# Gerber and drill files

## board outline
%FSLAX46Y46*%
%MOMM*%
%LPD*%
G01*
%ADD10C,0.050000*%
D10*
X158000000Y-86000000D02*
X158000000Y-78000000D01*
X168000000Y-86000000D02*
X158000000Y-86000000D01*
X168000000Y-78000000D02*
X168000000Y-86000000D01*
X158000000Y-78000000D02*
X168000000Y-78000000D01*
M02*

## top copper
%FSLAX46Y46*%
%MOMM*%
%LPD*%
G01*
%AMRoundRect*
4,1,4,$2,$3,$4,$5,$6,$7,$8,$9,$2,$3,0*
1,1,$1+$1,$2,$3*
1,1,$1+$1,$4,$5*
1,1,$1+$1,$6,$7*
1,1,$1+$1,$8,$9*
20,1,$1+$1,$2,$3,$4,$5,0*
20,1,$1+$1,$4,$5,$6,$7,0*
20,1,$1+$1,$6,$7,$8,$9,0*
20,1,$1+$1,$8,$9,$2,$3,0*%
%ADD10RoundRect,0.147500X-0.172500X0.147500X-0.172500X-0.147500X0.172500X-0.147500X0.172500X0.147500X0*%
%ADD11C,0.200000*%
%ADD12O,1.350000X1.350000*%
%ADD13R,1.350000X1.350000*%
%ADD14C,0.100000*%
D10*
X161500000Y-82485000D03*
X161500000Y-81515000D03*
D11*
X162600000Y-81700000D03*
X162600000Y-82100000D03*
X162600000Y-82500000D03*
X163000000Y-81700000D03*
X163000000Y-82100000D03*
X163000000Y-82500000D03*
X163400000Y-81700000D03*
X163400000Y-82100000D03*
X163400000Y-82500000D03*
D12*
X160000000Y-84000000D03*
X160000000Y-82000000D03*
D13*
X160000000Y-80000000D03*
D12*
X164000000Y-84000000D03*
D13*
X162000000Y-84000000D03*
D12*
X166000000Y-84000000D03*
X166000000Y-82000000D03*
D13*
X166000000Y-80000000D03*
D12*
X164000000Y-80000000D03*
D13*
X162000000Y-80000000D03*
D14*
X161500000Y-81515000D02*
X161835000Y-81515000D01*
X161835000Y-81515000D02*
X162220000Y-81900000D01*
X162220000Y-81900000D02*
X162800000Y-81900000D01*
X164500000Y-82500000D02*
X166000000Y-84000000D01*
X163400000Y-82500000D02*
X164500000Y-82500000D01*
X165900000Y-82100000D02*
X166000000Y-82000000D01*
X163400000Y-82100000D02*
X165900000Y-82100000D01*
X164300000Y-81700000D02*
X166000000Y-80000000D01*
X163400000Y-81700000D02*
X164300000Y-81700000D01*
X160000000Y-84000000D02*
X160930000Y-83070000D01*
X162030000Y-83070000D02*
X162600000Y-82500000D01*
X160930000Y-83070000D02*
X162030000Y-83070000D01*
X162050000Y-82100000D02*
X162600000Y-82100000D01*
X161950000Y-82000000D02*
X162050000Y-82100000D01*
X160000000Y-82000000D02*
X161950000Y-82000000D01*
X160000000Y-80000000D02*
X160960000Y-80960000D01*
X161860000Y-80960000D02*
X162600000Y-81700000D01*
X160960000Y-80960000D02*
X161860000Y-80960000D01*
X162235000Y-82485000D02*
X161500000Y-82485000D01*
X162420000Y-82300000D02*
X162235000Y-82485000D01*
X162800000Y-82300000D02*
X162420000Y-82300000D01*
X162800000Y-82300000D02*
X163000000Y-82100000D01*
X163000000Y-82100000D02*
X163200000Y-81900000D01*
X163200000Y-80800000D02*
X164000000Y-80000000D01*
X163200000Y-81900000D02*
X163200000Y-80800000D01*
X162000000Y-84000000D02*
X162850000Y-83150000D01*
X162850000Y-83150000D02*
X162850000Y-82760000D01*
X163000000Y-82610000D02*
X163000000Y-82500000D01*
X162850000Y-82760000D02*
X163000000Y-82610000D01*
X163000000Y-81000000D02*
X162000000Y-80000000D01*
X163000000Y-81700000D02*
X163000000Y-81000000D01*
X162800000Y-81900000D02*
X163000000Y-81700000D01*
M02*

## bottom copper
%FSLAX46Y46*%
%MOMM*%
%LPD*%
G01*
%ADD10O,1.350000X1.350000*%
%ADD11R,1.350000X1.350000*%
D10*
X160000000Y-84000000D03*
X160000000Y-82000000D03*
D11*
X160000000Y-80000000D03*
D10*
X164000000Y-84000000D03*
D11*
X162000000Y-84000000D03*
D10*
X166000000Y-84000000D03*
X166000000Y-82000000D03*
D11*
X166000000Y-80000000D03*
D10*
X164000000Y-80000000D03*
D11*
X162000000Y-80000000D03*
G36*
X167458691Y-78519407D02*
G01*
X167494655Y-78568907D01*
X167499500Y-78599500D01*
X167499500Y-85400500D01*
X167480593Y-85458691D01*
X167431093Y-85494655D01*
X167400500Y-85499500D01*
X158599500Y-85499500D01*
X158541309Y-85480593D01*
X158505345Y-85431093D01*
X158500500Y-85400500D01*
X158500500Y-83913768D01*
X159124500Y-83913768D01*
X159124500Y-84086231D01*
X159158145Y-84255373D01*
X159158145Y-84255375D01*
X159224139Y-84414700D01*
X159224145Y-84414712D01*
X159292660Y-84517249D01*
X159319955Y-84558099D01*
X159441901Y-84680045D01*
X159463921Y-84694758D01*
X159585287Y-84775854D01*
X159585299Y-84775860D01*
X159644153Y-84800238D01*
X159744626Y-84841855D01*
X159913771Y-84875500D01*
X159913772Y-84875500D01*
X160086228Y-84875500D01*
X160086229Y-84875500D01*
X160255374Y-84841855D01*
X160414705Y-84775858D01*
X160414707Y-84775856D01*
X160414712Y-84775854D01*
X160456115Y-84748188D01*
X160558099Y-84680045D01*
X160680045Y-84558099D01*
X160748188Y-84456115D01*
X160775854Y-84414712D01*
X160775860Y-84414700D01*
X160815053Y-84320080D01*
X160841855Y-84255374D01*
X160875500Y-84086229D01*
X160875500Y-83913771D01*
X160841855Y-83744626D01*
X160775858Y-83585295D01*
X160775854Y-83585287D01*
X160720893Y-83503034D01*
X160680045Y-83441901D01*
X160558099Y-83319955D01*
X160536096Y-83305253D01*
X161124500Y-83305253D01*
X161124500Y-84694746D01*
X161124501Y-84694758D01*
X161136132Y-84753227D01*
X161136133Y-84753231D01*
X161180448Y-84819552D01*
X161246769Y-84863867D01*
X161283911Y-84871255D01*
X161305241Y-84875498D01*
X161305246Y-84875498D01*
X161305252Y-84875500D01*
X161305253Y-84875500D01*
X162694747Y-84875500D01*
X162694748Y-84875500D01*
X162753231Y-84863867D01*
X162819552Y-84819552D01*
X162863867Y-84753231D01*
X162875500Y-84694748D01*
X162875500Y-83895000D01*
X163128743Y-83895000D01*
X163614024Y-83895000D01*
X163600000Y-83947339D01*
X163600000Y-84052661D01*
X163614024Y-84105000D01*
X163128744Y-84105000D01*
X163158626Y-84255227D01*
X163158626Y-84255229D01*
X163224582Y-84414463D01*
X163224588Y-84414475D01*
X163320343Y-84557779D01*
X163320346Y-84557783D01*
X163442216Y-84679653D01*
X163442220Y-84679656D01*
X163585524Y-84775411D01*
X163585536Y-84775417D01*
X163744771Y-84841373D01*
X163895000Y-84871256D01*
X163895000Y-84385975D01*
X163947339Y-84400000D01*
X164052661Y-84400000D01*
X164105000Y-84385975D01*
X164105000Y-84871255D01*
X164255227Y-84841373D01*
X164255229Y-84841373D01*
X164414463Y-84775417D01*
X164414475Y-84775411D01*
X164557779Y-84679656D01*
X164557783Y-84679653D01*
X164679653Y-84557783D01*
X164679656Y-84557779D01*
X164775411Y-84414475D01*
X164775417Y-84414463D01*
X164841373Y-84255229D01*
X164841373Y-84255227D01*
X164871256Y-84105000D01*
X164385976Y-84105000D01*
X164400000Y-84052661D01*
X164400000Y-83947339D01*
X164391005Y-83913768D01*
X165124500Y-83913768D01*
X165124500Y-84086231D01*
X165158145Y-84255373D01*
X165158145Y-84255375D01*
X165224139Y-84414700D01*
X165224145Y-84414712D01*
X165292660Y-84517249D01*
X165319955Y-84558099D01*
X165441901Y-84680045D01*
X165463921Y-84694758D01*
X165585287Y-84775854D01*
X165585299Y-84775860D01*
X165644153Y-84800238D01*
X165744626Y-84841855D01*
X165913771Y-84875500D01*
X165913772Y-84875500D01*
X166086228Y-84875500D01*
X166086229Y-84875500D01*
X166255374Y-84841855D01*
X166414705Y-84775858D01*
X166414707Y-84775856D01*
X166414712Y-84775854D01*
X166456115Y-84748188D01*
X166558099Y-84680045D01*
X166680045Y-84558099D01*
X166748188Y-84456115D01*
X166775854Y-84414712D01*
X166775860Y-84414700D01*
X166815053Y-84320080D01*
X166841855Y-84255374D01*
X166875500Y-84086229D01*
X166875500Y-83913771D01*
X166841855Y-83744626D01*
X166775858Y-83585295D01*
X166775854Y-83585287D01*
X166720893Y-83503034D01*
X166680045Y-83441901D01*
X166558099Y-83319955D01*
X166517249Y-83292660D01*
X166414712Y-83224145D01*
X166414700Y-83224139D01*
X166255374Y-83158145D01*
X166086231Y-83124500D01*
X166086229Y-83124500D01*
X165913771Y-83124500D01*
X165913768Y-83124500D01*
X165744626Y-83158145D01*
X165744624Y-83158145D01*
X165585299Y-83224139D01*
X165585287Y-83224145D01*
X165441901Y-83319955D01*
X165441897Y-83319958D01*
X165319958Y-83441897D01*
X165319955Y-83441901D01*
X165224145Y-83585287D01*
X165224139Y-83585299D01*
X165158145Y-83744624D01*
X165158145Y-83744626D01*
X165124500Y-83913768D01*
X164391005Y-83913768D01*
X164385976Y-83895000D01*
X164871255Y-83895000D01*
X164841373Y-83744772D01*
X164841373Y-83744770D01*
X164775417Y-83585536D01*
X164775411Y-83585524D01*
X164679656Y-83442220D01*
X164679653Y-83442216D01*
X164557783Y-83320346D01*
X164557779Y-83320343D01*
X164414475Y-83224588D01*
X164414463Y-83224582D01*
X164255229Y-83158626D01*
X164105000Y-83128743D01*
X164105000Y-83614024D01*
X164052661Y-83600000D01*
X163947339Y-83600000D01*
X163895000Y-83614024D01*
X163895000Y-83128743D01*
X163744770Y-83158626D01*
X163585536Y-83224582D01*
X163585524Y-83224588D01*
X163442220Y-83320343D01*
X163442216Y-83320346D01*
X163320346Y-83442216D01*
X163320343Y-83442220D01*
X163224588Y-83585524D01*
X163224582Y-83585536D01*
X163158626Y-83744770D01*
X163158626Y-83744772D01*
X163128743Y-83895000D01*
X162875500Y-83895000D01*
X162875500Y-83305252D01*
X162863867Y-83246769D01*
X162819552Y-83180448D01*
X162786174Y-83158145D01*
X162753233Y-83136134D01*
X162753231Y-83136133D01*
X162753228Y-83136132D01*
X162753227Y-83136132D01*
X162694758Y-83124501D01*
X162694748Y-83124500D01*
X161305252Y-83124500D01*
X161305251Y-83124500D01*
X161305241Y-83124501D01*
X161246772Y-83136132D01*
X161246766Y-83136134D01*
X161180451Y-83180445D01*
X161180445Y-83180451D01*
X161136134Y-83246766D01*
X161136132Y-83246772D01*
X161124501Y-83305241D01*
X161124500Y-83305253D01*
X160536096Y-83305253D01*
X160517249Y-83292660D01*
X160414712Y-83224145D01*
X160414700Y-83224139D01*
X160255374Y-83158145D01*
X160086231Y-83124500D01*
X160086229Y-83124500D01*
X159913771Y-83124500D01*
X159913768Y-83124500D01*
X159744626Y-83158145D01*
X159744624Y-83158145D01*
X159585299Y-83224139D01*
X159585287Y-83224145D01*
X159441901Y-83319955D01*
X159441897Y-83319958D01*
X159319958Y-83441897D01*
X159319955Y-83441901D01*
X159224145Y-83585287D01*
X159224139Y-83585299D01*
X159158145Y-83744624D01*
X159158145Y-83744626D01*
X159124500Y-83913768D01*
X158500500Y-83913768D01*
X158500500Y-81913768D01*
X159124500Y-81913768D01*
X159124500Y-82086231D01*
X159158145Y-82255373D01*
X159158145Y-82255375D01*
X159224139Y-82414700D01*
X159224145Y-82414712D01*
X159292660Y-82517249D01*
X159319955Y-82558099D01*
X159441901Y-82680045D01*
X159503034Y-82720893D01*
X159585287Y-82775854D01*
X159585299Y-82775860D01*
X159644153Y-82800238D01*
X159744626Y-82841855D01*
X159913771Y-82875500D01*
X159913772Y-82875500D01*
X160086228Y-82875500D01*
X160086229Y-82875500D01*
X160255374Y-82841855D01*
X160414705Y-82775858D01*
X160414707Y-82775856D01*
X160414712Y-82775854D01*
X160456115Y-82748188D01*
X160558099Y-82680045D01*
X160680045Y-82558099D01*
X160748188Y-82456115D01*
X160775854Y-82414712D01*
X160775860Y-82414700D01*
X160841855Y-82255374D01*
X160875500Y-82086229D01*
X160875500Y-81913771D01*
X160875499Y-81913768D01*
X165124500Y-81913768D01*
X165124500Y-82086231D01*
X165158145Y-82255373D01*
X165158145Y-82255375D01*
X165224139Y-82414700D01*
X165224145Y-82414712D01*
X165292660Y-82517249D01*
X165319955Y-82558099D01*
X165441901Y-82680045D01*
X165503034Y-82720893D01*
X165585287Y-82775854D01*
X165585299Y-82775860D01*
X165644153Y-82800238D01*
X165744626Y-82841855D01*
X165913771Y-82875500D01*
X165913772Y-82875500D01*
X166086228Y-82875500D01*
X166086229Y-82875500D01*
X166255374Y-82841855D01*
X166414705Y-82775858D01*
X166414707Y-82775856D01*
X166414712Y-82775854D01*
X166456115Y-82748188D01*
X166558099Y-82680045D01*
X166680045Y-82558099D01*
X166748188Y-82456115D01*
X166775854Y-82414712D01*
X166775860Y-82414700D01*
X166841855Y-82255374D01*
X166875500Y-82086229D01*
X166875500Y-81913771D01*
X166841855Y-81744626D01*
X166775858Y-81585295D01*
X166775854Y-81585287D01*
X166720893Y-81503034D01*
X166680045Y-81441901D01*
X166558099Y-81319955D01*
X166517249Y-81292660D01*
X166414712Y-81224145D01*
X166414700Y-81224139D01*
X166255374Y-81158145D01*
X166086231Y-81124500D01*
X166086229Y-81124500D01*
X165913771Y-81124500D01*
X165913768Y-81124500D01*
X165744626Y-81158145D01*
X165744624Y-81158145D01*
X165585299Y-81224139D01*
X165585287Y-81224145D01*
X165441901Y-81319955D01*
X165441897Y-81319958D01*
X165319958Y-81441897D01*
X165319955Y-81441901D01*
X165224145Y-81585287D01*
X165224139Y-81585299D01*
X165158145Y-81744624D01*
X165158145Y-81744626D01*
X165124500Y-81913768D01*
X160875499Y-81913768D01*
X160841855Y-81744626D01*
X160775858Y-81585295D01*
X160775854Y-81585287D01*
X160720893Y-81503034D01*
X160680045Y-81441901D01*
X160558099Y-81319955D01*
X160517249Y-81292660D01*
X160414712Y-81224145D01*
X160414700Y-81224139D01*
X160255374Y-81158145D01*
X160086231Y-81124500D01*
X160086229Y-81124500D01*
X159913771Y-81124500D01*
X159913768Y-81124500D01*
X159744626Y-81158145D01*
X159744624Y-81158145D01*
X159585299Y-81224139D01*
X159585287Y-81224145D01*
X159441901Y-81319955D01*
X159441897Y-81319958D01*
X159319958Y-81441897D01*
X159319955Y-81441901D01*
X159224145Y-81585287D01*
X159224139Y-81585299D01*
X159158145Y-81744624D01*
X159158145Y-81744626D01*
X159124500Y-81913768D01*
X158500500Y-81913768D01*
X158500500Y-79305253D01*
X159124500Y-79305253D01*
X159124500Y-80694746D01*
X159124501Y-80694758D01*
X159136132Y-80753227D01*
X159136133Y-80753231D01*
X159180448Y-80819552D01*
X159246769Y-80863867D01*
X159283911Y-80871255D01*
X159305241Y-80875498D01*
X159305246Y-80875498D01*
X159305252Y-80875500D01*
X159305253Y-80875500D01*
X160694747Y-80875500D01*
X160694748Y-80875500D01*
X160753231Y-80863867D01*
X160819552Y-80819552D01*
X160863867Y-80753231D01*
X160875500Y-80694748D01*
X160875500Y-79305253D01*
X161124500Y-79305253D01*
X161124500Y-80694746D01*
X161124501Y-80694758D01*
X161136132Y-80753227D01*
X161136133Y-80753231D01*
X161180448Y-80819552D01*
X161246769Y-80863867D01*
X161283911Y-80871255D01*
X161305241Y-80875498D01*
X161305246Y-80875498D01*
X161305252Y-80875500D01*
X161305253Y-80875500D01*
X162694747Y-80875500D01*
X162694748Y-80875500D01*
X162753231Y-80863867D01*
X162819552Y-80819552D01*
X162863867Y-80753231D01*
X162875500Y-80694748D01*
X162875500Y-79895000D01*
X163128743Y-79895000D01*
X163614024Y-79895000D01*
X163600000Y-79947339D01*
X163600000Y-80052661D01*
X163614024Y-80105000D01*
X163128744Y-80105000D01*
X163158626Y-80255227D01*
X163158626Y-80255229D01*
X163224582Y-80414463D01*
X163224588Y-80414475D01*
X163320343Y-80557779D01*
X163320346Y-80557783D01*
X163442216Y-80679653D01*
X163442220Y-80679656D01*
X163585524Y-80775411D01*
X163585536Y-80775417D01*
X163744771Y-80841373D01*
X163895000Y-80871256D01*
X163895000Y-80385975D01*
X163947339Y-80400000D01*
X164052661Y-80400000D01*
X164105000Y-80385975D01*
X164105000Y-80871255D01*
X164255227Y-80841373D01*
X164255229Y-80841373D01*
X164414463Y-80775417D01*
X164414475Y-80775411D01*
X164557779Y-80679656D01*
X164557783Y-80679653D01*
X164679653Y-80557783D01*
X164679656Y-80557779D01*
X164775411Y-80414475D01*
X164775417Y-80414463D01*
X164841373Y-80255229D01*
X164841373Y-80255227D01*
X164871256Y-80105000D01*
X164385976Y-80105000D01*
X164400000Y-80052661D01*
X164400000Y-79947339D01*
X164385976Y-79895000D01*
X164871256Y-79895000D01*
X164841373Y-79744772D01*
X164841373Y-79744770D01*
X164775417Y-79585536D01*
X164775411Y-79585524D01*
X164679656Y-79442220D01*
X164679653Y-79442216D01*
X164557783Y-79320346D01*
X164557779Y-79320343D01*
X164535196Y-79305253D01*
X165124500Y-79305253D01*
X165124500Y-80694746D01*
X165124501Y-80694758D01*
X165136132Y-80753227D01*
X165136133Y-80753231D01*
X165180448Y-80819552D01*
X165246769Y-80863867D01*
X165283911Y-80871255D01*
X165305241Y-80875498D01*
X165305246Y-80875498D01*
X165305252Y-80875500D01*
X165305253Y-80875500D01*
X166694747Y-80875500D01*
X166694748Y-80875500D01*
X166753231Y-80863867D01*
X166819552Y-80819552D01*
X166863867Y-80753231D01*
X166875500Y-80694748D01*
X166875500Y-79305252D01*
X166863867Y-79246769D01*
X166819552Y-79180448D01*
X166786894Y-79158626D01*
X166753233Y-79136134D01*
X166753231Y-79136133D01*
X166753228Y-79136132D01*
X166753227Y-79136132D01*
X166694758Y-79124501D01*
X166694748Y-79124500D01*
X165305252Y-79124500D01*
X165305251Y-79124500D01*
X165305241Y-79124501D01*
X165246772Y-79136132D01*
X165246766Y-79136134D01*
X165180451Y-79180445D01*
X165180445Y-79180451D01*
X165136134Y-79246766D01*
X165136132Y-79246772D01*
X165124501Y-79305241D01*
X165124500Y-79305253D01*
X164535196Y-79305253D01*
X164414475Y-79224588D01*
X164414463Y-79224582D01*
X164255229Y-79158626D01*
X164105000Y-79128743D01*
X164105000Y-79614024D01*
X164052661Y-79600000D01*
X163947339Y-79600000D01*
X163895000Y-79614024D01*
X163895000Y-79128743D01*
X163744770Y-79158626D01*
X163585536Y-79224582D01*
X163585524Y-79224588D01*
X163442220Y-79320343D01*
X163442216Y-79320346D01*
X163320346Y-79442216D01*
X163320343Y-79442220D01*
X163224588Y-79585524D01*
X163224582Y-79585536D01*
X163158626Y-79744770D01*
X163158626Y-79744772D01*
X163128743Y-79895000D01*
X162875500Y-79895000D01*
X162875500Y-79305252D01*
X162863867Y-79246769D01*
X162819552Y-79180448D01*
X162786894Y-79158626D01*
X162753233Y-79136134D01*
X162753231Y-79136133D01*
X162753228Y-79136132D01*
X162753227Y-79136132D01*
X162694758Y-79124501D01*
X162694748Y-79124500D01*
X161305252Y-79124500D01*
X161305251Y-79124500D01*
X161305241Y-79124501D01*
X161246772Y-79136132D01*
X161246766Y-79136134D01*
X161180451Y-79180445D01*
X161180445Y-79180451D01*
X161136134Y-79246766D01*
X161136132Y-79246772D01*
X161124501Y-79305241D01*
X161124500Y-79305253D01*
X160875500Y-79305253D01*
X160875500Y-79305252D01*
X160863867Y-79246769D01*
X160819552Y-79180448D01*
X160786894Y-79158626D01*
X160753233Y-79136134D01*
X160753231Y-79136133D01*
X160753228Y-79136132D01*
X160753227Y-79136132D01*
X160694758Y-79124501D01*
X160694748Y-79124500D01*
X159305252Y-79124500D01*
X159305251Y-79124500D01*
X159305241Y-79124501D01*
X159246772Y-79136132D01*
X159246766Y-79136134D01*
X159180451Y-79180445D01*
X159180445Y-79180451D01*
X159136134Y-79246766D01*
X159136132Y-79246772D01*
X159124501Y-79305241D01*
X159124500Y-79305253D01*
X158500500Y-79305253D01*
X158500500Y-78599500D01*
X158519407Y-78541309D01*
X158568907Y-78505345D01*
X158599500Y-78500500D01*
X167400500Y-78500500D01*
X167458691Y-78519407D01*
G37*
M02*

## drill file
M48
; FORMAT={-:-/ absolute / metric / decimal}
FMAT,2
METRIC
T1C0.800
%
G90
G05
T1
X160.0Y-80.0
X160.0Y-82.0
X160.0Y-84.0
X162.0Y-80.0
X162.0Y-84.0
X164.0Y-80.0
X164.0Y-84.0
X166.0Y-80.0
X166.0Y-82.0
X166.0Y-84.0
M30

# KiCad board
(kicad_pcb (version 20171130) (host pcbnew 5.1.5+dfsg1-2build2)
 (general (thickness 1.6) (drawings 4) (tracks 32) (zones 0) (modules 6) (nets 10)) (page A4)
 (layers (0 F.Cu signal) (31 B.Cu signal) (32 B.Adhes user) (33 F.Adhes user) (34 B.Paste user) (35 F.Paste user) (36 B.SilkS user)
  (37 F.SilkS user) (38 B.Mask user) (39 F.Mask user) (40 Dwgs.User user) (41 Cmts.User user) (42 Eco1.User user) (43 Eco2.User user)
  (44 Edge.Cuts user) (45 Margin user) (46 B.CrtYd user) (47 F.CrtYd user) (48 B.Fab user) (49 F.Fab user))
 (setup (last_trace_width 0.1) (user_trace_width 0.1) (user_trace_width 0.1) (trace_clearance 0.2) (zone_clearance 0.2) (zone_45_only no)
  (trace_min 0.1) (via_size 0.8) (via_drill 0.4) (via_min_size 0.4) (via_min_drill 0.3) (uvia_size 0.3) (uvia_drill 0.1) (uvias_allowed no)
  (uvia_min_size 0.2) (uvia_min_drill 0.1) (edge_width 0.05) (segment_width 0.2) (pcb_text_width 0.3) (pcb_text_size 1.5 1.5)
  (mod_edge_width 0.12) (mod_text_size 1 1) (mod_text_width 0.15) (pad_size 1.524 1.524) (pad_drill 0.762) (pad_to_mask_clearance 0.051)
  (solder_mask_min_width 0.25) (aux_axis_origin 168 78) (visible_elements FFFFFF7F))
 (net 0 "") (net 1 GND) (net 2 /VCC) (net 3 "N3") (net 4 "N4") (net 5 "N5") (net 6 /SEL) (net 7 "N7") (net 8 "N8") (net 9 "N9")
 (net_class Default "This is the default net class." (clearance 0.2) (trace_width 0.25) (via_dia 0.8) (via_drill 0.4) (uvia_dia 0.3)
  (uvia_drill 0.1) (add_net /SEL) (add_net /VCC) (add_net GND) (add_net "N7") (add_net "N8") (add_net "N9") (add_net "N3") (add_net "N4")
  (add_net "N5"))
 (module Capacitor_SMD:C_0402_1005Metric (layer F.Cu) (at 161.5 82 270)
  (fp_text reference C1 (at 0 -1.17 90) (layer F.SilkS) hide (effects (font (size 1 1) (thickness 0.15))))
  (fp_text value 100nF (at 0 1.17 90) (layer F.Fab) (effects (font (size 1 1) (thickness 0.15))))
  (pad 2 smd roundrect (at 0.485 0 270) (size 0.59 0.64) (layers F.Cu F.Paste F.Mask) (roundrect_rratio 0.25) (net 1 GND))
  (pad 1 smd roundrect (at -0.485 0 270) (size 0.59 0.64) (layers F.Cu F.Paste F.Mask) (roundrect_rratio 0.25) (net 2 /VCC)))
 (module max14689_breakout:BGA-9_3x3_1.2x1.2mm (layer F.Cu) (at 163 82.1 180)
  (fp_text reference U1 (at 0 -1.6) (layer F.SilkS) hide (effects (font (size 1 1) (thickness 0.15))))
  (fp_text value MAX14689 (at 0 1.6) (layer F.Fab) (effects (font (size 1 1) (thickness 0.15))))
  (pad C3 smd circle (at 0.4 0.4 180) (size 0.2 0.2) (layers F.Cu F.Paste F.Mask) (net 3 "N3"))
  (pad B3 smd circle (at 0.4 0 180) (size 0.2 0.2) (layers F.Cu F.Paste F.Mask) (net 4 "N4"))
  (pad A3 smd circle (at 0.4 -0.4 180) (size 0.2 0.2) (layers F.Cu F.Paste F.Mask) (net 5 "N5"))
  (pad C2 smd circle (at 0 0.4 180) (size 0.2 0.2) (layers F.Cu F.Paste F.Mask) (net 2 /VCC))
  (pad B2 smd circle (at 0 0 180) (size 0.2 0.2) (layers F.Cu F.Paste F.Mask) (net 1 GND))
  (pad A2 smd circle (at 0 -0.4 180) (size 0.2 0.2) (layers F.Cu F.Paste F.Mask) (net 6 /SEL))
  (pad C1 smd circle (at -0.4 0.4 180) (size 0.2 0.2) (layers F.Cu F.Paste F.Mask) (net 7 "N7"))
  (pad B1 smd circle (at -0.4 0 180) (size 0.2 0.2) (layers F.Cu F.Paste F.Mask) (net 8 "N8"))
  (pad A1 smd circle (at -0.4 -0.4 180) (size 0.2 0.2) (layers F.Cu F.Paste F.Mask) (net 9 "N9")))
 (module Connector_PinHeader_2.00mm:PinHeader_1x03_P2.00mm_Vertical (layer F.Cu) (at 160 80)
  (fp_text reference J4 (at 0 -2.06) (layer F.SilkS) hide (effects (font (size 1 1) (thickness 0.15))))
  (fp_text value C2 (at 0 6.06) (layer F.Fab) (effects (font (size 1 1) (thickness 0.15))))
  (pad 3 thru_hole oval (at 0 4) (size 1.35 1.35) (drill 0.8) (layers *.Cu *.Mask) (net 5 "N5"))
  (pad 2 thru_hole oval (at 0 2) (size 1.35 1.35) (drill 0.8) (layers *.Cu *.Mask) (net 4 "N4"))
  (pad 1 thru_hole rect (at 0 0) (size 1.35 1.35) (drill 0.8) (layers *.Cu *.Mask) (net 3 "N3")))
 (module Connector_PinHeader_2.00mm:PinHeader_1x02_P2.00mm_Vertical (layer F.Cu) (at 162 84 90)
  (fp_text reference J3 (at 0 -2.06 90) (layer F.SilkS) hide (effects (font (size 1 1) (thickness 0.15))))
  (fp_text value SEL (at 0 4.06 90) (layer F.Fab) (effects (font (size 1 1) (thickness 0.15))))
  (pad 2 thru_hole oval (at 0 2 90) (size 1.35 1.35) (drill 0.8) (layers *.Cu *.Mask) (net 1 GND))
  (pad 1 thru_hole rect (at 0 0 90) (size 1.35 1.35) (drill 0.8) (layers *.Cu *.Mask) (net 6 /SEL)))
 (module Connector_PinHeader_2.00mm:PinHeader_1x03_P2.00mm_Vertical (layer F.Cu) (at 166 80)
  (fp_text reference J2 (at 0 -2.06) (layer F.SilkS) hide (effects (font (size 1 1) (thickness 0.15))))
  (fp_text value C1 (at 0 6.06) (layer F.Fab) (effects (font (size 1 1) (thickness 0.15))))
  (pad 3 thru_hole oval (at 0 4) (size 1.35 1.35) (drill 0.8) (layers *.Cu *.Mask) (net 9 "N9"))
  (pad 2 thru_hole oval (at 0 2) (size 1.35 1.35) (drill 0.8) (layers *.Cu *.Mask) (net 8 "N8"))
  (pad 1 thru_hole rect (at 0 0) (size 1.35 1.35) (drill 0.8) (layers *.Cu *.Mask) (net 7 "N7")))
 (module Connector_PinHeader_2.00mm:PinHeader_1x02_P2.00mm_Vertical (layer F.Cu) (at 162 80 90)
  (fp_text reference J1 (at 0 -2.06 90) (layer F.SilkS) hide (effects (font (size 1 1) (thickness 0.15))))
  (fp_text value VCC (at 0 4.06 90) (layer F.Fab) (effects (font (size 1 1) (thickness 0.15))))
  (pad 2 thru_hole oval (at 0 2 90) (size 1.35 1.35) (drill 0.8) (layers *.Cu *.Mask) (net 1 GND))
  (pad 1 thru_hole rect (at 0 0 90) (size 1.35 1.35) (drill 0.8) (layers *.Cu *.Mask) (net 2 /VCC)))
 (gr_line (start 158 86) (end 158 78) (layer Edge.Cuts) (width 0.05))
 (gr_line (start 168 86) (end 158 86) (layer Edge.Cuts) (width 0.05))
 (gr_line (start 168 78) (end 168 86) (layer Edge.Cuts) (width 0.05))
 (gr_line (start 158 78) (end 168 78) (layer Edge.Cuts) (width 0.05))
 (segment (start 161.5 81.515) (end 161.835 81.515) (width 0.1) (layer F.Cu) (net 2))
 (segment (start 161.835 81.515) (end 162.22 81.9) (width 0.1) (layer F.Cu) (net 2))
 (segment (start 162.22 81.9) (end 162.8 81.9) (width 0.1) (layer F.Cu) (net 2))
 (segment (start 164.5 82.5) (end 166 84) (width 0.1) (layer F.Cu) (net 9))
 (segment (start 163.4 82.5) (end 164.5 82.5) (width 0.1) (layer F.Cu) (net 9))
 (segment (start 165.9 82.1) (end 166 82) (width 0.1) (layer F.Cu) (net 8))
 (segment (start 163.4 82.1) (end 165.9 82.1) (width 0.1) (layer F.Cu) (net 8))
 (segment (start 164.3 81.7) (end 166 80) (width 0.1) (layer F.Cu) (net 7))
 (segment (start 163.4 81.7) (end 164.3 81.7) (width 0.1) (layer F.Cu) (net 7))
 (segment (start 160 84) (end 160.93 83.07) (width 0.1) (layer F.Cu) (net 5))
 (segment (start 162.03 83.07) (end 162.6 82.5) (width 0.1) (layer F.Cu) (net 5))
 (segment (start 160.93 83.07) (end 162.03 83.07) (width 0.1) (layer F.Cu) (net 5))
 (segment (start 162.05 82.1) (end 162.6 82.1) (width 0.1) (layer F.Cu) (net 4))
 (segment (start 161.95 82) (end 162.05 82.1) (width 0.1) (layer F.Cu) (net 4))
 (segment (start 160 82) (end 161.95 82) (width 0.1) (layer F.Cu) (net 4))
 (segment (start 160 80) (end 160.96 80.96) (width 0.1) (layer F.Cu) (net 3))
 (segment (start 161.86 80.96) (end 162.6 81.7) (width 0.1) (layer F.Cu) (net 3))
 (segment (start 160.96 80.96) (end 161.86 80.96) (width 0.1) (layer F.Cu) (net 3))
 (segment (start 162.235 82.485) (end 161.5 82.485) (width 0.1) (layer F.Cu) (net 1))
 (segment (start 162.42 82.3) (end 162.235 82.485) (width 0.1) (layer F.Cu) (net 1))
 (segment (start 162.8 82.3) (end 162.42 82.3) (width 0.1) (layer F.Cu) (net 1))
 (segment (start 162.8 82.3) (end 163 82.1) (width 0.1) (layer F.Cu) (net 1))
 (segment (start 163 82.1) (end 163.2 81.9) (width 0.1) (layer F.Cu) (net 1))
 (segment (start 163.2 80.8) (end 164 80) (width 0.1) (layer F.Cu) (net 1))
 (segment (start 163.2 81.9) (end 163.2 80.8) (width 0.1) (layer F.Cu) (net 1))
 (segment (start 162 84) (end 162.85 83.15) (width 0.1) (layer F.Cu) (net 6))
 (segment (start 162.85 83.15) (end 162.85 82.76) (width 0.1) (layer F.Cu) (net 6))
 (segment (start 163 82.61) (end 163 82.5) (width 0.1) (layer F.Cu) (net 6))
 (segment (start 162.85 82.76) (end 163 82.61) (width 0.1) (layer F.Cu) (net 6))
 (segment (start 163 81) (end 162 80) (width 0.1) (layer F.Cu) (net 2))
 (segment (start 163 81.7) (end 163 81) (width 0.1) (layer F.Cu) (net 2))
 (segment (start 162.8 81.9) (end 163 81.7) (width 0.1) (layer F.Cu) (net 2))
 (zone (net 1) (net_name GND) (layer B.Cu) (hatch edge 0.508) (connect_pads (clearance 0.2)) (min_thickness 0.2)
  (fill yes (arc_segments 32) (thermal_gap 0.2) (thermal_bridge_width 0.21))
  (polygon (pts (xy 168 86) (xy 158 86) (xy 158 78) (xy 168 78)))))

